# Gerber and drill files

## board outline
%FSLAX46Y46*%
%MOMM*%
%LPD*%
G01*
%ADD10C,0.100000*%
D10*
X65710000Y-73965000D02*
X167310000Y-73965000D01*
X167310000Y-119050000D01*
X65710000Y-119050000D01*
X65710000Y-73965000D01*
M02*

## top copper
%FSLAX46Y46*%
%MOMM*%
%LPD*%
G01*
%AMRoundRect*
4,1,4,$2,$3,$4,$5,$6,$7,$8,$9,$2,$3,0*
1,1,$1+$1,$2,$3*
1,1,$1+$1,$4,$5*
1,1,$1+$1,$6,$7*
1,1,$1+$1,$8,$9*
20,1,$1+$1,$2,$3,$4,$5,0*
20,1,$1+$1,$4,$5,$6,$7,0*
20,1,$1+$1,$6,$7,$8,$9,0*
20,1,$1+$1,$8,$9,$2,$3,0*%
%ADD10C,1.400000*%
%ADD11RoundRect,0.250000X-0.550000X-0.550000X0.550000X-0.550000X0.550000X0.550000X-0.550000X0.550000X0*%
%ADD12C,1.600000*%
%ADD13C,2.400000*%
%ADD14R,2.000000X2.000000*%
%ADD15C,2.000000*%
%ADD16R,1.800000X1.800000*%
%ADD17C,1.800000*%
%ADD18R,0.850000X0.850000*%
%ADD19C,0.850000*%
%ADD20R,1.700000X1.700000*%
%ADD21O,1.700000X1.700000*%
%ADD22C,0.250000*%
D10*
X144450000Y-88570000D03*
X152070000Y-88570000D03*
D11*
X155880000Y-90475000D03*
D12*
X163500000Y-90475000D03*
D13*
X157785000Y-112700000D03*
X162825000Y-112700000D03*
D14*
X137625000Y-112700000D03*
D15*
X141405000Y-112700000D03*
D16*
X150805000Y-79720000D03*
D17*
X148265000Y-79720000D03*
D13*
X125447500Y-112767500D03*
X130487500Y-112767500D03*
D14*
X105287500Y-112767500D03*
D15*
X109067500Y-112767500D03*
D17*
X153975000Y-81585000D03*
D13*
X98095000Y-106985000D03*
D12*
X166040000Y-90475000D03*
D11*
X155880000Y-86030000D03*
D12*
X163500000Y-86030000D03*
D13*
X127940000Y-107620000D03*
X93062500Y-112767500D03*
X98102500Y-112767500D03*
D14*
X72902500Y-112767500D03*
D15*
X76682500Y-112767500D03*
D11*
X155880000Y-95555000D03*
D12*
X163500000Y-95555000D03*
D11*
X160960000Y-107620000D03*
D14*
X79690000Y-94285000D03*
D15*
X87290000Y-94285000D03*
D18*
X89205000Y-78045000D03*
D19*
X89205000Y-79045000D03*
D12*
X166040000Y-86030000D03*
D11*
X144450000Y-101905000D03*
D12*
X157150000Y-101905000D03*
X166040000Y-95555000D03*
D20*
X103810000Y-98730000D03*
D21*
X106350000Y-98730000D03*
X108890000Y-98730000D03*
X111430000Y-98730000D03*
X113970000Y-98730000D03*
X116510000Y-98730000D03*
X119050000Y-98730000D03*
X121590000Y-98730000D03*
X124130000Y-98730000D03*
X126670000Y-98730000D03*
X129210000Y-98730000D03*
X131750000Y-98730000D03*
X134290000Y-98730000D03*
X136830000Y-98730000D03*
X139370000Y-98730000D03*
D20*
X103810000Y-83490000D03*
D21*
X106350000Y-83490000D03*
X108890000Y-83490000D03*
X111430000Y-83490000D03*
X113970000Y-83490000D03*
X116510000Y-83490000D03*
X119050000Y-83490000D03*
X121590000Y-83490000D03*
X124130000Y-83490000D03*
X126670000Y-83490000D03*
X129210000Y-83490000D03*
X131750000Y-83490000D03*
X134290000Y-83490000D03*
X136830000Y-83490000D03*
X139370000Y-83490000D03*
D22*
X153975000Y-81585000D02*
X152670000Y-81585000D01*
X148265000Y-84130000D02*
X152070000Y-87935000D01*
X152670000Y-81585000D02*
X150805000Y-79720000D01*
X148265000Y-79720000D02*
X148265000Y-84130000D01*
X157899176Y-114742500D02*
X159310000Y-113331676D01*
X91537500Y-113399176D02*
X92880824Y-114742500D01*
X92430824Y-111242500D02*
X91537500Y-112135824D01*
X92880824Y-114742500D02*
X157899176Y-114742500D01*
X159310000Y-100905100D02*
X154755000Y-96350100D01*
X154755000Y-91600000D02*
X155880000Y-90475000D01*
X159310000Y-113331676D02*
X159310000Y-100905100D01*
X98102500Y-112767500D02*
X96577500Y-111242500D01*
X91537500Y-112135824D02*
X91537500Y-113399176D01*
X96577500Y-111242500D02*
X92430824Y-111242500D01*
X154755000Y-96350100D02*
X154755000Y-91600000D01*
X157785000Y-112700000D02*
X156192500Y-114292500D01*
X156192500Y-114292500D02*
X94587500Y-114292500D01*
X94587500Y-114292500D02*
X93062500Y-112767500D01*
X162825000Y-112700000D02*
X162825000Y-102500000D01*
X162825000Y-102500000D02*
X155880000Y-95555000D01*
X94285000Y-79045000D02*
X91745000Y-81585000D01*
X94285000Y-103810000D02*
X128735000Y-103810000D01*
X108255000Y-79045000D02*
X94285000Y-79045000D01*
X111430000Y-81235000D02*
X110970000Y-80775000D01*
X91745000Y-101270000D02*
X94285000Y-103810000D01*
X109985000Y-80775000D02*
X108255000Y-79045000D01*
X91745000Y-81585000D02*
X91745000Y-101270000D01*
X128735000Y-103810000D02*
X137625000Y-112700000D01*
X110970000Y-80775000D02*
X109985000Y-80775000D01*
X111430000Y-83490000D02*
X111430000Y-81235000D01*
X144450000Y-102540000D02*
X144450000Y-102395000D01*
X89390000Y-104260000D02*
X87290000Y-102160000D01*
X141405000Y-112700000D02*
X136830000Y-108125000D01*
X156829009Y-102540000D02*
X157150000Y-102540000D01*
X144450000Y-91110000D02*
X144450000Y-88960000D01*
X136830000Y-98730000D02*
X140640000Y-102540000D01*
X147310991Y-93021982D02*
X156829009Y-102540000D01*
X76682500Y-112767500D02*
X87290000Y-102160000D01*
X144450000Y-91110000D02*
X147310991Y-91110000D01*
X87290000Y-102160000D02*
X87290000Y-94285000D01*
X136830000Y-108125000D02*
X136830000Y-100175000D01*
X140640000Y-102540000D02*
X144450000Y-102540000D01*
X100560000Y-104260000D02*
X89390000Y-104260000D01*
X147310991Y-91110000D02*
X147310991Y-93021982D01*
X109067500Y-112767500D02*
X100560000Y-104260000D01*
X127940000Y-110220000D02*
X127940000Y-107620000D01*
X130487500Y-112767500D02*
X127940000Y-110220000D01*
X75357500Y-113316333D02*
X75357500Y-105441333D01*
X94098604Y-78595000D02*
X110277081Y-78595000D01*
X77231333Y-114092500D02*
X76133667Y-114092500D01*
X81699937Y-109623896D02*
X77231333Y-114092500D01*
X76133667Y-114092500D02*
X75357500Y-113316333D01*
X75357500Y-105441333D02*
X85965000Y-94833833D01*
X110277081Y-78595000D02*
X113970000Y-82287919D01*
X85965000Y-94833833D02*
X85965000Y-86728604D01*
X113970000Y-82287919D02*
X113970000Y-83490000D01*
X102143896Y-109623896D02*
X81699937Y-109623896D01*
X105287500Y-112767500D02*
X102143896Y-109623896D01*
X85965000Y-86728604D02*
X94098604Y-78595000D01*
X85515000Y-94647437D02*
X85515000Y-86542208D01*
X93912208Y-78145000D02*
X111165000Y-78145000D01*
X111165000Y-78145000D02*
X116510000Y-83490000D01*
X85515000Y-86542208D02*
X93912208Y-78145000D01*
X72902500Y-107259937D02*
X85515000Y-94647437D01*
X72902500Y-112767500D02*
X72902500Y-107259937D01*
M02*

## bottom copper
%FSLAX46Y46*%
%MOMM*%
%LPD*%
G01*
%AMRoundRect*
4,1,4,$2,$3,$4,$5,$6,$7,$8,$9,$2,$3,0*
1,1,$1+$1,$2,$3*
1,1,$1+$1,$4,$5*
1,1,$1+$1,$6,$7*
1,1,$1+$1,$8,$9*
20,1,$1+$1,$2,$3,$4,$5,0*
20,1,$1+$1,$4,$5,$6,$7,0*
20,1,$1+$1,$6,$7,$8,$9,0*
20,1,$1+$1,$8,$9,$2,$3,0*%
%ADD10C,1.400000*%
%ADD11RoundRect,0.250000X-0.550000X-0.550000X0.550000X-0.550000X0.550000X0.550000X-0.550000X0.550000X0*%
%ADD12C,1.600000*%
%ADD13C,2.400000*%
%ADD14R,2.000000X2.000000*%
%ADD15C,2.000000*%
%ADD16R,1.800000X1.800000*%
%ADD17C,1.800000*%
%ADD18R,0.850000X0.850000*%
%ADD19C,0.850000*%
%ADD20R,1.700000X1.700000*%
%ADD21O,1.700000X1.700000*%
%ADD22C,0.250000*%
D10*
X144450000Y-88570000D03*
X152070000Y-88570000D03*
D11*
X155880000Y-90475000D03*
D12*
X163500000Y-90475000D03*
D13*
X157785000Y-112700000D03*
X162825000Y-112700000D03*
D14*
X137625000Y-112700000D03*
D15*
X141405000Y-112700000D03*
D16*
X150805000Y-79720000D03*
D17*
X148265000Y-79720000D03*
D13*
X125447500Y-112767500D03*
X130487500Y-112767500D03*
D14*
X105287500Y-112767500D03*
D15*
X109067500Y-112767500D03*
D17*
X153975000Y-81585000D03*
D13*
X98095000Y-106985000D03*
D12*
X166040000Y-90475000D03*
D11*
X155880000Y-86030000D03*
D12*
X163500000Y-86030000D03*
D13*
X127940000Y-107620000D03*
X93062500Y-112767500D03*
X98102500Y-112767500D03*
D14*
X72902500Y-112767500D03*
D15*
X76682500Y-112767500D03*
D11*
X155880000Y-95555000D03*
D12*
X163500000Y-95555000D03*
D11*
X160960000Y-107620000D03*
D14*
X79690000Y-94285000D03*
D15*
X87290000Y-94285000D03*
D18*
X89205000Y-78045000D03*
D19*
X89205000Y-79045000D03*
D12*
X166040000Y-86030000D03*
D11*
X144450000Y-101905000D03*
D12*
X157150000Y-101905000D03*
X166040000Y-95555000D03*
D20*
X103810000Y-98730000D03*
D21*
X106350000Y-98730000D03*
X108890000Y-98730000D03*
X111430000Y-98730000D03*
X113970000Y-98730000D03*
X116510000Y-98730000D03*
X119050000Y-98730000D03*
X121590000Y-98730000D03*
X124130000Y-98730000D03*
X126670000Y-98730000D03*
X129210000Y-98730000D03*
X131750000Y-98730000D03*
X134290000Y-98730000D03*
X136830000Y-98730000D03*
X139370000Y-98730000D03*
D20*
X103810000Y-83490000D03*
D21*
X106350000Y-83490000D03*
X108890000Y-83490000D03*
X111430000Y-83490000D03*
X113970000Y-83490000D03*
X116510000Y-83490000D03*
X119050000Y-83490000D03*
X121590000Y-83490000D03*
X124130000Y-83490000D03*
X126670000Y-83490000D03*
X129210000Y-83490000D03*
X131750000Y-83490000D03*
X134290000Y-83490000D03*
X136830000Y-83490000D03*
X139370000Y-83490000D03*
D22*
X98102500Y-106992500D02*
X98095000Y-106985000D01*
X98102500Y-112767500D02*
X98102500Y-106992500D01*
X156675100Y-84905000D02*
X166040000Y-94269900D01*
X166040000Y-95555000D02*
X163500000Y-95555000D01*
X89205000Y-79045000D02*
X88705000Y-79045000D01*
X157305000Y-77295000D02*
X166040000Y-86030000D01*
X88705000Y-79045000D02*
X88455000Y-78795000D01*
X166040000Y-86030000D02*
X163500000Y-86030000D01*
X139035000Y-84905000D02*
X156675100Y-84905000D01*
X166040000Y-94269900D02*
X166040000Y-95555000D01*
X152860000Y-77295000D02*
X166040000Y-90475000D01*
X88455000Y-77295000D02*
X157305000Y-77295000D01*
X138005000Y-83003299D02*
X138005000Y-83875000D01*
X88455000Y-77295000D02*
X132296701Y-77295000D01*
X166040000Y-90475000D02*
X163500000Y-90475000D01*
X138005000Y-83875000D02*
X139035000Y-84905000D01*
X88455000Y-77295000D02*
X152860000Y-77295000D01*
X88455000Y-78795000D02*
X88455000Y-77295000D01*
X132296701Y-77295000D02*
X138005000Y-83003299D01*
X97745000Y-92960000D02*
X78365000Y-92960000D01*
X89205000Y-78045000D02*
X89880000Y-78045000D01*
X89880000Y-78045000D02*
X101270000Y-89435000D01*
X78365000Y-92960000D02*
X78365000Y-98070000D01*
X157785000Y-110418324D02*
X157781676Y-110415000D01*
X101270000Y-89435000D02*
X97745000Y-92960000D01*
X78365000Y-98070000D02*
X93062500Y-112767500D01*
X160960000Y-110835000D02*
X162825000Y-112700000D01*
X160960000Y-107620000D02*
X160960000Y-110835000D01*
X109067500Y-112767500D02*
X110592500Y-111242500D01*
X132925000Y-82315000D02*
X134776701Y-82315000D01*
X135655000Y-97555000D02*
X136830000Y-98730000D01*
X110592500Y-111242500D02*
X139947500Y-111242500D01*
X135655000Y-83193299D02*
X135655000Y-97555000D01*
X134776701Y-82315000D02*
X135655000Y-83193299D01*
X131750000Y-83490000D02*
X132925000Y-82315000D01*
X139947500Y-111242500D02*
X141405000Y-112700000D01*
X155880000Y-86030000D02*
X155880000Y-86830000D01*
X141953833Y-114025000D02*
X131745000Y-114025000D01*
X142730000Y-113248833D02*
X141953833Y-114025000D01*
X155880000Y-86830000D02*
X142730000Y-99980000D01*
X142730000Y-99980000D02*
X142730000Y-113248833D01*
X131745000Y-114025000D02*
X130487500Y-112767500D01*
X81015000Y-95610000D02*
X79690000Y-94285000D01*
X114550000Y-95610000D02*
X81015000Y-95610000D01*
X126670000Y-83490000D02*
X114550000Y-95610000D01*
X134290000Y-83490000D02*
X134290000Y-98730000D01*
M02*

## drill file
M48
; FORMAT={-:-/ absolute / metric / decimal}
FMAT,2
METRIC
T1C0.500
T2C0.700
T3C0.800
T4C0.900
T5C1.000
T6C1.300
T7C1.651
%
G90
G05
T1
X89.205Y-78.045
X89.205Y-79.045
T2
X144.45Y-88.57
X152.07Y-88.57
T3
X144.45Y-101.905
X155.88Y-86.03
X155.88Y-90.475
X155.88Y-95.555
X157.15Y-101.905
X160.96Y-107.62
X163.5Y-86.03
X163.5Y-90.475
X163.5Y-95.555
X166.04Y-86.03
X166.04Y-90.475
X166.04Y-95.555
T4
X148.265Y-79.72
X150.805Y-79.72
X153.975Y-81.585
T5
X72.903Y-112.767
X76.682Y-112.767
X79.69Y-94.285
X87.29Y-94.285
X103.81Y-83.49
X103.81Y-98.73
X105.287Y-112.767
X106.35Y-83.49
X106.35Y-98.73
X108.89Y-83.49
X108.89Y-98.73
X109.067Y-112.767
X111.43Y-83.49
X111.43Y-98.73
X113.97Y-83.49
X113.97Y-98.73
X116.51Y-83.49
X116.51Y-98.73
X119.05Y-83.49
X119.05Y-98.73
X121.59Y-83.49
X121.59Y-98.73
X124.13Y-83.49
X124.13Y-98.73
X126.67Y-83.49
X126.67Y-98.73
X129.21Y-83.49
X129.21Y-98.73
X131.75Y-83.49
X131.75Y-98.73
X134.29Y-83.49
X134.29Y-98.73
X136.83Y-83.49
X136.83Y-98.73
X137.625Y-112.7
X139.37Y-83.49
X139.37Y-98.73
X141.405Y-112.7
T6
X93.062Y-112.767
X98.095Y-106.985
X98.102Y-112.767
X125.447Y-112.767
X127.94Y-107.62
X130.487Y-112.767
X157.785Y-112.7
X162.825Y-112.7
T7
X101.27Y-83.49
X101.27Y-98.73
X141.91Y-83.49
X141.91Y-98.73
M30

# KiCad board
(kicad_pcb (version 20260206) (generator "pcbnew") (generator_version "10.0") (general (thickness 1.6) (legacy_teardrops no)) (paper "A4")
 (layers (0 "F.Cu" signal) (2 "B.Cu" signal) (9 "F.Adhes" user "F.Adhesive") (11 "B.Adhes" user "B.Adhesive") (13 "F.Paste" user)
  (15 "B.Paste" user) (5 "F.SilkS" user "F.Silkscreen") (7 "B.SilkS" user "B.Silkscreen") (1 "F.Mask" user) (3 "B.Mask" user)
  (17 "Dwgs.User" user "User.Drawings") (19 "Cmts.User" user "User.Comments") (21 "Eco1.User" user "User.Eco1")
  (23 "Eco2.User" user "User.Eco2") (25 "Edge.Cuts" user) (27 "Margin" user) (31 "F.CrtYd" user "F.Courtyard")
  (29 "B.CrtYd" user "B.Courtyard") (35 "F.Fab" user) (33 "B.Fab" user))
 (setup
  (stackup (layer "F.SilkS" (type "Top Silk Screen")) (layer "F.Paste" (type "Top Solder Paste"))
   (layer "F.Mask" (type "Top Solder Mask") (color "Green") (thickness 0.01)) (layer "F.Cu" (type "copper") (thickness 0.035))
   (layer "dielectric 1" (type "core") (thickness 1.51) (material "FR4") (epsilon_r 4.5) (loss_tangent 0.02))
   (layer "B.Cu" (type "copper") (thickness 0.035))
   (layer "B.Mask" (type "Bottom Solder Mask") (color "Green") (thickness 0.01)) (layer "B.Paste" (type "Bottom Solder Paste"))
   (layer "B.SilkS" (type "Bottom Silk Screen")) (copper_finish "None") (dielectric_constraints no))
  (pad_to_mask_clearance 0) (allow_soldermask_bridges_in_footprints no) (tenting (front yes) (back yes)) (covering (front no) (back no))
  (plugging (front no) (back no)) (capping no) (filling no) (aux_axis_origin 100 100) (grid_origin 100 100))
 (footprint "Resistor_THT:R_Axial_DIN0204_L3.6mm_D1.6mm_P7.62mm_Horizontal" (layer "F.Cu") (at 144.45 88.57)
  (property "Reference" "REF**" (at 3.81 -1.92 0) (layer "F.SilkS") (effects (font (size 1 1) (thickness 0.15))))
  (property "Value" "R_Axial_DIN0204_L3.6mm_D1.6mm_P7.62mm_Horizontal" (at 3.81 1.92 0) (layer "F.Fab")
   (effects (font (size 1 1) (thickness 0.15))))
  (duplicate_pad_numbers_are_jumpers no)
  (pad "1" thru_hole circle (at 0 0) (size 1.4 1.4) (drill 0.7) (layers "*.Cu" "*.Mask") (remove_unused_layers no))
  (pad "2" thru_hole circle (at 7.62 0) (size 1.4 1.4) (drill 0.7) (layers "*.Cu" "*.Mask") (remove_unused_layers no)))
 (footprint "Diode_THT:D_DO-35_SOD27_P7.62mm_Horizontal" (layer "F.Cu") (at 155.88 90.475)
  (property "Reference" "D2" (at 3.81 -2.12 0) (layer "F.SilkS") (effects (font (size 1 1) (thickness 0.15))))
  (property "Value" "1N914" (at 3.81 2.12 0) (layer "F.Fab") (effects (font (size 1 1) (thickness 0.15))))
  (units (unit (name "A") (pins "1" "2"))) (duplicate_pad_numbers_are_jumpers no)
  (pad "1" thru_hole roundrect (at 0 0) (size 1.6 1.6) (drill 0.8) (layers "*.Cu" "*.Mask") (remove_unused_layers no)
   (roundrect_rratio 0.15625) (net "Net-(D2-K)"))
  (pad "2" thru_hole circle (at 7.62 0) (size 1.6 1.6) (drill 0.8) (layers "*.Cu" "*.Mask") (remove_unused_layers no) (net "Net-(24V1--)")))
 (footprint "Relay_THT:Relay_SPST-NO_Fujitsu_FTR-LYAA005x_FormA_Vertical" (layer "F.Cu") (at 137.625 112.7)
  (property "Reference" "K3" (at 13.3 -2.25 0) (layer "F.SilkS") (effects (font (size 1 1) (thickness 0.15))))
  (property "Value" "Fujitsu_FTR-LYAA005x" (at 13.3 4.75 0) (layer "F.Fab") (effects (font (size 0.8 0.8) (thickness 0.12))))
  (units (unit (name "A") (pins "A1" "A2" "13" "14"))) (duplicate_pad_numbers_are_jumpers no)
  (pad "13" thru_hole circle (at 20.16 0) (size 2.4 2.4) (drill 1.3) (layers "*.Cu" "*.Mask") (remove_unused_layers no) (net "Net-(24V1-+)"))
  (pad "14" thru_hole circle (at 25.2 0) (size 2.4 2.4) (drill 1.3) (layers "*.Cu" "*.Mask") (remove_unused_layers no) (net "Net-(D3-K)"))
  (pad "A1" thru_hole rect (at 0 0) (size 2 2) (drill 1) (layers "*.Cu" "*.Mask") (remove_unused_layers no) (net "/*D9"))
  (pad "A2" thru_hole circle (at 3.78 0) (size 2 2) (drill 1) (layers "*.Cu" "*.Mask") (remove_unused_layers no) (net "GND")))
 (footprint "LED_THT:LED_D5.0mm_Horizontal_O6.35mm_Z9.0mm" (layer "F.Cu") (at 150.805 79.72 180)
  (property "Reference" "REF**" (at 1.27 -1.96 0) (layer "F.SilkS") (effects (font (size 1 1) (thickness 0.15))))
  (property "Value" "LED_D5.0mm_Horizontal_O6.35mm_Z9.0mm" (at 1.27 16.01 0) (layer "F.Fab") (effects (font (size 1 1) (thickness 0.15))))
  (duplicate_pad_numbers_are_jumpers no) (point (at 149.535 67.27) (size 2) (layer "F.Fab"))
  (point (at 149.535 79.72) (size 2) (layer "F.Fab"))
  (pad "1" thru_hole rect (at 0 0 180) (size 1.8 1.8) (drill 0.9) (layers "*.Cu" "*.Mask") (remove_unused_layers no))
  (pad "2" thru_hole circle (at 2.54 0 180) (size 1.8 1.8) (drill 0.9) (layers "*.Cu" "*.Mask") (remove_unused_layers no)))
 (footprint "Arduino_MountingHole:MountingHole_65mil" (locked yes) (layer "F.Cu") (at 101.27 83.49)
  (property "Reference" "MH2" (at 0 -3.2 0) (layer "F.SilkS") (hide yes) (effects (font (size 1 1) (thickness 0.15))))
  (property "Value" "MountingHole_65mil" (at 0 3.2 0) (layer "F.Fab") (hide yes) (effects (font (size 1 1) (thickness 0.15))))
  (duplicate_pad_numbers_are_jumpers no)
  (pad "" np_thru_hole circle (at 0 0) (size 1.651 1.651) (drill 1.651) (layers "*.Cu" "*.Mask")))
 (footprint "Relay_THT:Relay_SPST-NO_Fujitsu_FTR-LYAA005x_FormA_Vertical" (layer "F.Cu") (at 105.2875 112.7675)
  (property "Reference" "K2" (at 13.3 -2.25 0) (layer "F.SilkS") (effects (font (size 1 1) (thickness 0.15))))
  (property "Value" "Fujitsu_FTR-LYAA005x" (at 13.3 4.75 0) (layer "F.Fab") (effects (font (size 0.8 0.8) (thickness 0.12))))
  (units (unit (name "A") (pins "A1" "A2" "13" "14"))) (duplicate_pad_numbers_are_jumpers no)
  (pad "13" thru_hole circle (at 20.16 0) (size 2.4 2.4) (drill 1.3) (layers "*.Cu" "*.Mask") (remove_unused_layers no)
   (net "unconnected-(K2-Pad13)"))
  (pad "14" thru_hole circle (at 25.2 0) (size 2.4 2.4) (drill 1.3) (layers "*.Cu" "*.Mask") (remove_unused_layers no) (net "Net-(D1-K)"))
  (pad "A1" thru_hole rect (at 0 0) (size 2 2) (drill 1) (layers "*.Cu" "*.Mask") (remove_unused_layers no) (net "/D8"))
  (pad "A2" thru_hole circle (at 3.78 0) (size 2 2) (drill 1) (layers "*.Cu" "*.Mask") (remove_unused_layers no) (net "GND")))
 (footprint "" (layer "F.Cu") (at 153.975 81.585)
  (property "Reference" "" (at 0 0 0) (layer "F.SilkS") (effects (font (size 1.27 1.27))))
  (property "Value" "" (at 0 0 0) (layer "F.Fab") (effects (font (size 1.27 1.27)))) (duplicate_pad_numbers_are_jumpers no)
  (pad "2" thru_hole circle (at 0 0 180) (size 1.8 1.8) (drill 0.9) (layers "*.Cu" "*.Mask") (remove_unused_layers no)))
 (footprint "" (layer "F.Cu") (at 98.095 106.985)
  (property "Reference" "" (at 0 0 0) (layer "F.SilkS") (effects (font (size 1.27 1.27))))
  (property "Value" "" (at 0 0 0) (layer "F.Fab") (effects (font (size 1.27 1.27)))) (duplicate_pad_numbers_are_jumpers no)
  (pad "14" thru_hole circle (at 0 0) (size 2.4 2.4) (drill 1.3) (layers "*.Cu" "*.Mask") (remove_unused_layers no) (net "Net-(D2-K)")))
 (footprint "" (layer "F.Cu") (at 166.04 90.475)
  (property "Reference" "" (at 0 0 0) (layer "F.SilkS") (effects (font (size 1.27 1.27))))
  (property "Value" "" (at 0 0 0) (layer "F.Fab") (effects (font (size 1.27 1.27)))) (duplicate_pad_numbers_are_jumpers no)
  (pad "2" thru_hole circle (at 0 0) (size 1.6 1.6) (drill 0.8) (layers "*.Cu" "*.Mask") (remove_unused_layers no) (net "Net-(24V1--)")))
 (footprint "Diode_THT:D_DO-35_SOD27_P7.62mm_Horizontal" (layer "F.Cu") (at 155.88 86.03)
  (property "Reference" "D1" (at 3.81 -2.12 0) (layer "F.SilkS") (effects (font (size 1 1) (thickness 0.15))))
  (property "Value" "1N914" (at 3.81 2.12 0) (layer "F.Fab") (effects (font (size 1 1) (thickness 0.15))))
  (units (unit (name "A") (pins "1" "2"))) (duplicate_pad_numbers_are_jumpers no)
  (pad "1" thru_hole roundrect (at 0 0) (size 1.6 1.6) (drill 0.8) (layers "*.Cu" "*.Mask") (remove_unused_layers no)
   (roundrect_rratio 0.15625) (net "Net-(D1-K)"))
  (pad "2" thru_hole circle (at 7.62 0) (size 1.6 1.6) (drill 0.8) (layers "*.Cu" "*.Mask") (remove_unused_layers no) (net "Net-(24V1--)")))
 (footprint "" (layer "F.Cu") (at 127.94 107.62)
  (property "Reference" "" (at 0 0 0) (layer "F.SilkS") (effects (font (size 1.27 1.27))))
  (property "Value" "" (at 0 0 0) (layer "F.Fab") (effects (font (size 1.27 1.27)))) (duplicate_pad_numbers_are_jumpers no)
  (pad "14" thru_hole circle (at 0 0) (size 2.4 2.4) (drill 1.3) (layers "*.Cu" "*.Mask") (remove_unused_layers no) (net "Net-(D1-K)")))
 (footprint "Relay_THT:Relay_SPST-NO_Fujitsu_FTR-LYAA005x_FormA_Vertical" (layer "F.Cu") (at 72.9025 112.7675)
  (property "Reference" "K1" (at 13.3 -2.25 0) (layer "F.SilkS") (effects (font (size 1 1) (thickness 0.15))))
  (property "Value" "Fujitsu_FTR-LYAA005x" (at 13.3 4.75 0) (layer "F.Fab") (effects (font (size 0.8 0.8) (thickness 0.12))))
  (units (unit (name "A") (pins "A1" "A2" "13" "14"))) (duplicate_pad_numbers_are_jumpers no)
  (pad "13" thru_hole circle (at 20.16 0) (size 2.4 2.4) (drill 1.3) (layers "*.Cu" "*.Mask") (remove_unused_layers no) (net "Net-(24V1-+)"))
  (pad "14" thru_hole circle (at 25.2 0) (size 2.4 2.4) (drill 1.3) (layers "*.Cu" "*.Mask") (remove_unused_layers no) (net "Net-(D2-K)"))
  (pad "A1" thru_hole rect (at 0 0) (size 2 2) (drill 1) (layers "*.Cu" "*.Mask") (remove_unused_layers no) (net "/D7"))
  (pad "A2" thru_hole circle (at 3.78 0) (size 2 2) (drill 1) (layers "*.Cu" "*.Mask") (remove_unused_layers no) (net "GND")))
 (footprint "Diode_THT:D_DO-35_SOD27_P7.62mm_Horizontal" (layer "F.Cu") (at 155.88 95.555)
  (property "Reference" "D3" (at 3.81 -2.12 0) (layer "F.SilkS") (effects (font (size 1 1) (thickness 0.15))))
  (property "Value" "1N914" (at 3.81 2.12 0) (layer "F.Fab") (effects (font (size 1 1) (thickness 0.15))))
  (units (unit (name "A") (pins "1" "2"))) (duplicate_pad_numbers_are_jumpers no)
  (pad "1" thru_hole roundrect (at 0 0) (size 1.6 1.6) (drill 0.8) (layers "*.Cu" "*.Mask") (remove_unused_layers no)
   (roundrect_rratio 0.15625) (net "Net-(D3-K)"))
  (pad "2" thru_hole circle (at 7.62 0) (size 1.6 1.6) (drill 0.8) (layers "*.Cu" "*.Mask") (remove_unused_layers no) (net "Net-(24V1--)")))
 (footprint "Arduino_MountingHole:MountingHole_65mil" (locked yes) (layer "F.Cu") (at 141.91 98.73)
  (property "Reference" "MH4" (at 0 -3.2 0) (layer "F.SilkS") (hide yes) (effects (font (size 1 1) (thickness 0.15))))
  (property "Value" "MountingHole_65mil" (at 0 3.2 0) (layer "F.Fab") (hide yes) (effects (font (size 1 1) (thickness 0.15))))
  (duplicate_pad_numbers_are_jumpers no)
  (pad "" np_thru_hole circle (at 0 0) (size 1.651 1.651) (drill 1.651) (layers "*.Cu" "*.Mask")))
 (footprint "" (layer "F.Cu") (at 160.96 107.62)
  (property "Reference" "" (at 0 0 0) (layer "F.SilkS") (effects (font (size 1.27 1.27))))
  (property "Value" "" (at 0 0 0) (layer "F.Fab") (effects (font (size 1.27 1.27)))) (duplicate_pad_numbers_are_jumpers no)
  (pad "1" thru_hole roundrect (at 0 0) (size 1.6 1.6) (drill 0.8) (layers "*.Cu" "*.Mask") (remove_unused_layers no)
   (roundrect_rratio 0.15625) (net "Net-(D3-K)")))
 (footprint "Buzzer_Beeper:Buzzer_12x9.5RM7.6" (layer "F.Cu") (at 79.69 94.285)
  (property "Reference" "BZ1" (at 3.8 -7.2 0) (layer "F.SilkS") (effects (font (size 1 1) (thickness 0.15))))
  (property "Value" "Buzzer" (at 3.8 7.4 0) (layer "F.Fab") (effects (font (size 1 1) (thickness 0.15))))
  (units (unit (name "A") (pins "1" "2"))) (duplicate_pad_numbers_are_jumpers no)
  (pad "1" thru_hole rect (at 0 0) (size 2 2) (drill 1) (layers "*.Cu" "*.Mask") (remove_unused_layers no) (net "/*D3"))
  (pad "2" thru_hole circle (at 7.6 0) (size 2 2) (drill 1) (layers "*.Cu" "*.Mask") (remove_unused_layers no) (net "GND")))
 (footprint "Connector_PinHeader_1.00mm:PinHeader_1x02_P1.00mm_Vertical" (layer "F.Cu") (at 89.205 78.045)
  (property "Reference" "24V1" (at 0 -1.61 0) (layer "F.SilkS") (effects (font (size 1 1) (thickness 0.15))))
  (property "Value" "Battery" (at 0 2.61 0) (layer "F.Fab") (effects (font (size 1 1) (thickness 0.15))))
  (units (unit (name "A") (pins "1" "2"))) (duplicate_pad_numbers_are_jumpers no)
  (pad "1" thru_hole rect (at 0 0) (size 0.85 0.85) (drill 0.5) (layers "*.Cu" "*.Mask") (remove_unused_layers no) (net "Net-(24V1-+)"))
  (pad "2" thru_hole circle (at 0 1) (size 0.85 0.85) (drill 0.5) (layers "*.Cu" "*.Mask") (remove_unused_layers no) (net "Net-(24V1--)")))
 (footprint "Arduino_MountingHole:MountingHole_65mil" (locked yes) (layer "F.Cu") (at 101.27 98.73)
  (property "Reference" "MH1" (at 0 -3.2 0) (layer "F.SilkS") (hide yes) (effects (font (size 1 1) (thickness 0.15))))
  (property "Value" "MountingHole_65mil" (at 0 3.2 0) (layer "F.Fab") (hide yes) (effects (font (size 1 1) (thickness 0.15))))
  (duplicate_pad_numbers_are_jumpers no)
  (pad "" np_thru_hole circle (at 0 0) (size 1.651 1.651) (drill 1.651) (layers "*.Cu" "*.Mask")))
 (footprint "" (layer "F.Cu") (at 166.04 86.03)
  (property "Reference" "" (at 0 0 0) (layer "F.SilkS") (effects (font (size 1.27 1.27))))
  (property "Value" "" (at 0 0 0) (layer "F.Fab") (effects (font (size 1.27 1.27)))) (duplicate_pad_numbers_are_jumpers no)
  (pad "2" thru_hole circle (at 0 0) (size 1.6 1.6) (drill 0.8) (layers "*.Cu" "*.Mask") (remove_unused_layers no) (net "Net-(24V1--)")))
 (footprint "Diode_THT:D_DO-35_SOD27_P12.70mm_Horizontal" (layer "F.Cu") (at 144.45 101.905)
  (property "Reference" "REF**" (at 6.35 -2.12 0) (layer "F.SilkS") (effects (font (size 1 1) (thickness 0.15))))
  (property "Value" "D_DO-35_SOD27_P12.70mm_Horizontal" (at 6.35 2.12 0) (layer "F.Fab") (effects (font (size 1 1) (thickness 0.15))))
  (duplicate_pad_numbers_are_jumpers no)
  (pad "1" thru_hole roundrect (at 0 0) (size 1.6 1.6) (drill 0.8) (layers "*.Cu" "*.Mask") (remove_unused_layers no)
   (roundrect_rratio 0.15625))
  (pad "2" thru_hole circle (at 12.7 0) (size 1.6 1.6) (drill 0.8) (layers "*.Cu" "*.Mask") (remove_unused_layers no)))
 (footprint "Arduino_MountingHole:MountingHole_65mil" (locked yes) (layer "F.Cu") (at 141.91 83.49)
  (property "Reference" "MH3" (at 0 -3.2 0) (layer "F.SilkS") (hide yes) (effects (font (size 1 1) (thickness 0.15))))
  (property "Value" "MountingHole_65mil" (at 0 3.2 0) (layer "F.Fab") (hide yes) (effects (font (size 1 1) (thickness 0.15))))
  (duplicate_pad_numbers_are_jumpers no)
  (pad "" np_thru_hole circle (at 0 0) (size 1.651 1.651) (drill 1.651) (layers "*.Cu" "*.Mask")))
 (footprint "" (layer "F.Cu") (at 166.04 95.555)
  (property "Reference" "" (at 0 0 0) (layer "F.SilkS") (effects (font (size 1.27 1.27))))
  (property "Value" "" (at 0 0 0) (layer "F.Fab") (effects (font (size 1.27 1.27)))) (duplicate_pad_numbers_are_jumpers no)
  (pad "2" thru_hole circle (at 0 0) (size 1.6 1.6) (drill 0.8) (layers "*.Cu" "*.Mask") (remove_unused_layers no) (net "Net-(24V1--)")))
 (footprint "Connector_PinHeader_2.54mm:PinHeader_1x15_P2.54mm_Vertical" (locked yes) (layer "B.Cu") (at 103.81 98.73 -90)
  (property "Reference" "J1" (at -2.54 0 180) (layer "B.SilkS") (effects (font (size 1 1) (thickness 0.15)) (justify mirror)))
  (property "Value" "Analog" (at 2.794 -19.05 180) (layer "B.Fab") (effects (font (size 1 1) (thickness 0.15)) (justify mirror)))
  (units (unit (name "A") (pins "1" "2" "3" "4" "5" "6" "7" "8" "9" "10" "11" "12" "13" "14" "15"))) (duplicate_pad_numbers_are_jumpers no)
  (pad "1" thru_hole rect (at 0 0 270) (size 1.7 1.7) (drill 1) (layers "*.Cu" "*.Mask") (remove_unused_layers no) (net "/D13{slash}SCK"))
  (pad "2" thru_hole oval (at 0 -2.54 270) (size 1.7 1.7) (drill 1) (layers "*.Cu" "*.Mask") (remove_unused_layers no) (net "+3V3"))
  (pad "3" thru_hole oval (at 0 -5.08 270) (size 1.7 1.7) (drill 1) (layers "*.Cu" "*.Mask") (remove_unused_layers no) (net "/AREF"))
  (pad "4" thru_hole oval (at 0 -7.62 270) (size 1.7 1.7) (drill 1) (layers "*.Cu" "*.Mask") (remove_unused_layers no) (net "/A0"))
  (pad "5" thru_hole oval (at 0 -10.16 270) (size 1.7 1.7) (drill 1) (layers "*.Cu" "*.Mask") (remove_unused_layers no) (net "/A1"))
  (pad "6" thru_hole oval (at 0 -12.7 270) (size 1.7 1.7) (drill 1) (layers "*.Cu" "*.Mask") (remove_unused_layers no) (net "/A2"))
  (pad "7" thru_hole oval (at 0 -15.24 270) (size 1.7 1.7) (drill 1) (layers "*.Cu" "*.Mask") (remove_unused_layers no) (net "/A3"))
  (pad "8" thru_hole oval (at 0 -17.78 270) (size 1.7 1.7) (drill 1) (layers "*.Cu" "*.Mask") (remove_unused_layers no)
   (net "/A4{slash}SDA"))
  (pad "9" thru_hole oval (at 0 -20.32 270) (size 1.7 1.7) (drill 1) (layers "*.Cu" "*.Mask") (remove_unused_layers no)
   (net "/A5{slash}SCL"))
  (pad "10" thru_hole oval (at 0 -22.86 270) (size 1.7 1.7) (drill 1) (layers "*.Cu" "*.Mask") (remove_unused_layers no) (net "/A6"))
  (pad "11" thru_hole oval (at 0 -25.4 270) (size 1.7 1.7) (drill 1) (layers "*.Cu" "*.Mask") (remove_unused_layers no) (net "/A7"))
  (pad "12" thru_hole oval (at 0 -27.94 270) (size 1.7 1.7) (drill 1) (layers "*.Cu" "*.Mask") (remove_unused_layers no) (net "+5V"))
  (pad "13" thru_hole oval (at 0 -30.48 270) (size 1.7 1.7) (drill 1) (layers "*.Cu" "*.Mask") (remove_unused_layers no) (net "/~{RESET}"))
  (pad "14" thru_hole oval (at 0 -33.02 270) (size 1.7 1.7) (drill 1) (layers "*.Cu" "*.Mask") (remove_unused_layers no) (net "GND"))
  (pad "15" thru_hole oval (at 0 -35.56 270) (size 1.7 1.7) (drill 1) (layers "*.Cu" "*.Mask") (remove_unused_layers no) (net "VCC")))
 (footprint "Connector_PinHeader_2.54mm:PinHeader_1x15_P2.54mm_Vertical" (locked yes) (layer "B.Cu") (at 103.81 83.49 -90)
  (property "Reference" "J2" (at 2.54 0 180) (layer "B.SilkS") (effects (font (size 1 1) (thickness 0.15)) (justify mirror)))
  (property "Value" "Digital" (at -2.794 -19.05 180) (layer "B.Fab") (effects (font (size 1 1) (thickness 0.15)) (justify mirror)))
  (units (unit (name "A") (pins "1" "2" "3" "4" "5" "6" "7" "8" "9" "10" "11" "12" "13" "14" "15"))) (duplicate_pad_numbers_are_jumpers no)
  (pad "1" thru_hole rect (at 0 0 270) (size 1.7 1.7) (drill 1) (layers "*.Cu" "*.Mask") (remove_unused_layers no) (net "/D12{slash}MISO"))
  (pad "2" thru_hole oval (at 0 -2.54 270) (size 1.7 1.7) (drill 1) (layers "*.Cu" "*.Mask") (remove_unused_layers no)
   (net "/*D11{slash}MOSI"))
  (pad "3" thru_hole oval (at 0 -5.08 270) (size 1.7 1.7) (drill 1) (layers "*.Cu" "*.Mask") (remove_unused_layers no)
   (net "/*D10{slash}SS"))
  (pad "4" thru_hole oval (at 0 -7.62 270) (size 1.7 1.7) (drill 1) (layers "*.Cu" "*.Mask") (remove_unused_layers no) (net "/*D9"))
  (pad "5" thru_hole oval (at 0 -10.16 270) (size 1.7 1.7) (drill 1) (layers "*.Cu" "*.Mask") (remove_unused_layers no) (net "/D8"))
  (pad "6" thru_hole oval (at 0 -12.7 270) (size 1.7 1.7) (drill 1) (layers "*.Cu" "*.Mask") (remove_unused_layers no) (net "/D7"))
  (pad "7" thru_hole oval (at 0 -15.24 270) (size 1.7 1.7) (drill 1) (layers "*.Cu" "*.Mask") (remove_unused_layers no) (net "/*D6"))
  (pad "8" thru_hole oval (at 0 -17.78 270) (size 1.7 1.7) (drill 1) (layers "*.Cu" "*.Mask") (remove_unused_layers no) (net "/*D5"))
  (pad "9" thru_hole oval (at 0 -20.32 270) (size 1.7 1.7) (drill 1) (layers "*.Cu" "*.Mask") (remove_unused_layers no) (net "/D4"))
  (pad "10" thru_hole oval (at 0 -22.86 270) (size 1.7 1.7) (drill 1) (layers "*.Cu" "*.Mask") (remove_unused_layers no) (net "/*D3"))
  (pad "11" thru_hole oval (at 0 -25.4 270) (size 1.7 1.7) (drill 1) (layers "*.Cu" "*.Mask") (remove_unused_layers no) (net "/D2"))
  (pad "12" thru_hole oval (at 0 -27.94 270) (size 1.7 1.7) (drill 1) (layers "*.Cu" "*.Mask") (remove_unused_layers no) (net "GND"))
  (pad "13" thru_hole oval (at 0 -30.48 270) (size 1.7 1.7) (drill 1) (layers "*.Cu" "*.Mask") (remove_unused_layers no) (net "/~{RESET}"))
  (pad "14" thru_hole oval (at 0 -33.02 270) (size 1.7 1.7) (drill 1) (layers "*.Cu" "*.Mask") (remove_unused_layers no)
   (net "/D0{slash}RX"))
  (pad "15" thru_hole oval (at 0 -35.56 270) (size 1.7 1.7) (drill 1) (layers "*.Cu" "*.Mask") (remove_unused_layers no)
   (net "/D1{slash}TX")))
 (gr_rect (start 65.71 73.965) (end 167.31 119.05) (stroke (width 0.1) (type default)) (fill no) (layer "Edge.Cuts"))
 (segment (start 153.975 81.585) (end 152.67 81.585) (width 0.25) (layer "F.Cu") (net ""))
 (segment (start 148.265 84.13) (end 152.07 87.935) (width 0.25) (layer "F.Cu") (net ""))
 (segment (start 152.67 81.585) (end 150.805 79.72) (width 0.25) (layer "F.Cu") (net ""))
 (segment (start 148.265 79.72) (end 148.265 84.13) (width 0.25) (layer "F.Cu") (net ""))
 (segment (start 157.899176 114.7425) (end 159.31 113.331676) (width 0.25) (layer "F.Cu") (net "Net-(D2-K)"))
 (segment (start 91.5375 113.399176) (end 92.880824 114.7425) (width 0.25) (layer "F.Cu") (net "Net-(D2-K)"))
 (segment (start 92.430824 111.2425) (end 91.5375 112.135824) (width 0.25) (layer "F.Cu") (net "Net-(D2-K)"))
 (segment (start 92.880824 114.7425) (end 157.899176 114.7425) (width 0.25) (layer "F.Cu") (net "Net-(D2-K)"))
 (segment (start 159.31 100.9051) (end 154.755 96.3501) (width 0.25) (layer "F.Cu") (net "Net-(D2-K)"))
 (segment (start 154.755 91.6) (end 155.88 90.475) (width 0.25) (layer "F.Cu") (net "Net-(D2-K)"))
 (segment (start 159.31 113.331676) (end 159.31 100.9051) (width 0.25) (layer "F.Cu") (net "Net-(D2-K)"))
 (segment (start 98.1025 112.7675) (end 96.5775 111.2425) (width 0.25) (layer "F.Cu") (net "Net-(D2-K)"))
 (segment (start 91.5375 112.135824) (end 91.5375 113.399176) (width 0.25) (layer "F.Cu") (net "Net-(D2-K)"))
 (segment (start 96.5775 111.2425) (end 92.430824 111.2425) (width 0.25) (layer "F.Cu") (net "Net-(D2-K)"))
 (segment (start 154.755 96.3501) (end 154.755 91.6) (width 0.25) (layer "F.Cu") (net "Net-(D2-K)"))
 (segment (start 98.1025 106.9925) (end 98.095 106.985) (width 0.25) (layer "B.Cu") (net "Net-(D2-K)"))
 (segment (start 98.1025 112.7675) (end 98.1025 106.9925) (width 0.25) (layer "B.Cu") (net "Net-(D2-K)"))
 (segment (start 156.6751 84.905) (end 166.04 94.2699) (width 0.25) (layer "B.Cu") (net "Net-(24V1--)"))
 (segment (start 166.04 95.555) (end 163.5 95.555) (width 0.25) (layer "B.Cu") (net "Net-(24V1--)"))
 (segment (start 89.205 79.045) (end 88.705 79.045) (width 0.25) (layer "B.Cu") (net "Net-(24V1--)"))
 (segment (start 157.305 77.295) (end 166.04 86.03) (width 0.25) (layer "B.Cu") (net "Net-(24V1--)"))
 (segment (start 88.705 79.045) (end 88.455 78.795) (width 0.25) (layer "B.Cu") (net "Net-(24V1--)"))
 (segment (start 166.04 86.03) (end 163.5 86.03) (width 0.25) (layer "B.Cu") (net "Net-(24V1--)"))
 (segment (start 139.035 84.905) (end 156.6751 84.905) (width 0.25) (layer "B.Cu") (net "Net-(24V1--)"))
 (segment (start 166.04 94.2699) (end 166.04 95.555) (width 0.25) (layer "B.Cu") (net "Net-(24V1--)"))
 (segment (start 152.86 77.295) (end 166.04 90.475) (width 0.25) (layer "B.Cu") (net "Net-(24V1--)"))
 (segment (start 88.455 77.295) (end 157.305 77.295) (width 0.25) (layer "B.Cu") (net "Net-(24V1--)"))
 (segment (start 138.005 83.003299) (end 138.005 83.875) (width 0.25) (layer "B.Cu") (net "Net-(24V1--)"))
 (segment (start 88.455 77.295) (end 132.296701 77.295) (width 0.25) (layer "B.Cu") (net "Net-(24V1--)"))
 (segment (start 166.04 90.475) (end 163.5 90.475) (width 0.25) (layer "B.Cu") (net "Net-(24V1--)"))
 (segment (start 138.005 83.875) (end 139.035 84.905) (width 0.25) (layer "B.Cu") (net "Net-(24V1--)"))
 (segment (start 88.455 77.295) (end 152.86 77.295) (width 0.25) (layer "B.Cu") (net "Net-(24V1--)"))
 (segment (start 88.455 78.795) (end 88.455 77.295) (width 0.25) (layer "B.Cu") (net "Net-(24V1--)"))
 (segment (start 132.296701 77.295) (end 138.005 83.003299) (width 0.25) (layer "B.Cu") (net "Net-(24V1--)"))
 (segment (start 157.785 112.7) (end 156.1925 114.2925) (width 0.25) (layer "F.Cu") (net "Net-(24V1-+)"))
 (segment (start 156.1925 114.2925) (end 94.5875 114.2925) (width 0.25) (layer "F.Cu") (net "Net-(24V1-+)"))
 (segment (start 94.5875 114.2925) (end 93.0625 112.7675) (width 0.25) (layer "F.Cu") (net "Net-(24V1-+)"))
 (segment (start 97.745 92.96) (end 78.365 92.96) (width 0.25) (layer "B.Cu") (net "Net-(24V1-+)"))
 (segment (start 89.205 78.045) (end 89.88 78.045) (width 0.25) (layer "B.Cu") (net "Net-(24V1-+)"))
 (segment (start 89.88 78.045) (end 101.27 89.435) (width 0.25) (layer "B.Cu") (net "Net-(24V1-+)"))
 (segment (start 78.365 92.96) (end 78.365 98.07) (width 0.25) (layer "B.Cu") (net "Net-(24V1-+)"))
 (segment (start 157.785 110.418324) (end 157.781676 110.415) (width 0.25) (layer "B.Cu") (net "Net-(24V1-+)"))
 (segment (start 101.27 89.435) (end 97.745 92.96) (width 0.25) (layer "B.Cu") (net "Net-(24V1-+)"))
 (segment (start 78.365 98.07) (end 93.0625 112.7675) (width 0.25) (layer "B.Cu") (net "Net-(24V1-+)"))
 (segment (start 162.825 112.7) (end 162.825 102.5) (width 0.25) (layer "F.Cu") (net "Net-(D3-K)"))
 (segment (start 162.825 102.5) (end 155.88 95.555) (width 0.25) (layer "F.Cu") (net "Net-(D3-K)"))
 (segment (start 160.96 110.835) (end 162.825 112.7) (width 0.25) (layer "B.Cu") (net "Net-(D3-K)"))
 (segment (start 160.96 107.62) (end 160.96 110.835) (width 0.25) (layer "B.Cu") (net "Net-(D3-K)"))
 (segment (start 94.285 79.045) (end 91.745 81.585) (width 0.25) (layer "F.Cu") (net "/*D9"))
 (segment (start 94.285 103.81) (end 128.735 103.81) (width 0.25) (layer "F.Cu") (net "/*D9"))
 (segment (start 108.255 79.045) (end 94.285 79.045) (width 0.25) (layer "F.Cu") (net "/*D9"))
 (segment (start 111.43 81.235) (end 110.97 80.775) (width 0.25) (layer "F.Cu") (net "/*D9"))
 (segment (start 91.745 101.27) (end 94.285 103.81) (width 0.25) (layer "F.Cu") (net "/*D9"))
 (segment (start 109.985 80.775) (end 108.255 79.045) (width 0.25) (layer "F.Cu") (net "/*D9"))
 (segment (start 91.745 81.585) (end 91.745 101.27) (width 0.25) (layer "F.Cu") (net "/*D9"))
 (segment (start 128.735 103.81) (end 137.625 112.7) (width 0.25) (layer "F.Cu") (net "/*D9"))
 (segment (start 110.97 80.775) (end 109.985 80.775) (width 0.25) (layer "F.Cu") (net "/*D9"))
 (segment (start 111.43 83.49) (end 111.43 81.235) (width 0.25) (layer "F.Cu") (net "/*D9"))
 (segment (start 144.45 102.54) (end 144.45 102.395) (width 0.25) (layer "F.Cu") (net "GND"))
 (segment (start 89.39 104.26) (end 87.29 102.16) (width 0.25) (layer "F.Cu") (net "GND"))
 (segment (start 141.405 112.7) (end 136.83 108.125) (width 0.25) (layer "F.Cu") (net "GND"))
 (segment (start 156.829009 102.54) (end 157.15 102.54) (width 0.25) (layer "F.Cu") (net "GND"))
 (segment (start 144.45 91.11) (end 144.45 88.96) (width 0.25) (layer "F.Cu") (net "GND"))
 (segment (start 136.83 98.73) (end 140.64 102.54) (width 0.25) (layer "F.Cu") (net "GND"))
 (segment (start 147.310991 93.021982) (end 156.829009 102.54) (width 0.25) (layer "F.Cu") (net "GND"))
 (segment (start 76.6825 112.7675) (end 87.29 102.16) (width 0.25) (layer "F.Cu") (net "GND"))
 (segment (start 144.45 91.11) (end 147.310991 91.11) (width 0.25) (layer "F.Cu") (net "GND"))
 (segment (start 87.29 102.16) (end 87.29 94.285) (width 0.25) (layer "F.Cu") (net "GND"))
 (segment (start 136.83 108.125) (end 136.83 100.175) (width 0.25) (layer "F.Cu") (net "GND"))
 (segment (start 140.64 102.54) (end 144.45 102.54) (width 0.25) (layer "F.Cu") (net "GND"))
 (segment (start 100.56 104.26) (end 89.39 104.26) (width 0.25) (layer "F.Cu") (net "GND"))
 (segment (start 147.310991 91.11) (end 147.310991 93.021982) (width 0.25) (layer "F.Cu") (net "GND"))
 (segment (start 109.0675 112.7675) (end 100.56 104.26) (width 0.25) (layer "F.Cu") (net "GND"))
 (segment (start 109.0675 112.7675) (end 110.5925 111.2425) (width 0.25) (layer "B.Cu") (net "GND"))
 (segment (start 132.925 82.315) (end 134.776701 82.315) (width 0.25) (layer "B.Cu") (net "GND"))
 (segment (start 135.655 97.555) (end 136.83 98.73) (width 0.25) (layer "B.Cu") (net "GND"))
 (segment (start 110.5925 111.2425) (end 139.9475 111.2425) (width 0.25) (layer "B.Cu") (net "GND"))
 (segment (start 135.655 83.193299) (end 135.655 97.555) (width 0.25) (layer "B.Cu") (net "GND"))
 (segment (start 134.776701 82.315) (end 135.655 83.193299) (width 0.25) (layer "B.Cu") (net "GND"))
 (segment (start 131.75 83.49) (end 132.925 82.315) (width 0.25) (layer "B.Cu") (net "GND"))
 (segment (start 139.9475 111.2425) (end 141.405 112.7) (width 0.25) (layer "B.Cu") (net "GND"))
 (segment (start 127.94 110.22) (end 127.94 107.62) (width 0.25) (layer "F.Cu") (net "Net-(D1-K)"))
 (segment (start 130.4875 112.7675) (end 127.94 110.22) (width 0.25) (layer "F.Cu") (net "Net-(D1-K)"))
 (segment (start 155.88 86.03) (end 155.88 86.83) (width 0.25) (layer "B.Cu") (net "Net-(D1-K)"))
 (segment (start 141.953833 114.025) (end 131.745 114.025) (width 0.25) (layer "B.Cu") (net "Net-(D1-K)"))
 (segment (start 142.73 113.248833) (end 141.953833 114.025) (width 0.25) (layer "B.Cu") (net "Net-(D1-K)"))
 (segment (start 155.88 86.83) (end 142.73 99.98) (width 0.25) (layer "B.Cu") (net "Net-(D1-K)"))
 (segment (start 142.73 99.98) (end 142.73 113.248833) (width 0.25) (layer "B.Cu") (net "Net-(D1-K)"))
 (segment (start 131.745 114.025) (end 130.4875 112.7675) (width 0.25) (layer "B.Cu") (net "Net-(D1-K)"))
 (segment (start 75.3575 113.316333) (end 75.3575 105.441333) (width 0.25) (layer "F.Cu") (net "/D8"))
 (segment (start 94.098604 78.595) (end 110.277081 78.595) (width 0.25) (layer "F.Cu") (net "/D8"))
 (segment (start 77.231333 114.0925) (end 76.133667 114.0925) (width 0.25) (layer "F.Cu") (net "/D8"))
 (segment (start 81.699937 109.623896) (end 77.231333 114.0925) (width 0.25) (layer "F.Cu") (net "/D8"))
 (segment (start 76.133667 114.0925) (end 75.3575 113.316333) (width 0.25) (layer "F.Cu") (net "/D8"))
 (segment (start 75.3575 105.441333) (end 85.965 94.833833) (width 0.25) (layer "F.Cu") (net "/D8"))
 (segment (start 110.277081 78.595) (end 113.97 82.287919) (width 0.25) (layer "F.Cu") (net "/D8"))
 (segment (start 85.965 94.833833) (end 85.965 86.728604) (width 0.25) (layer "F.Cu") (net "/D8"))
 (segment (start 113.97 82.287919) (end 113.97 83.49) (width 0.25) (layer "F.Cu") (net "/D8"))
 (segment (start 102.143896 109.623896) (end 81.699937 109.623896) (width 0.25) (layer "F.Cu") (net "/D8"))
 (segment (start 105.2875 112.7675) (end 102.143896 109.623896) (width 0.25) (layer "F.Cu") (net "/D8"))
 (segment (start 85.965 86.728604) (end 94.098604 78.595) (width 0.25) (layer "F.Cu") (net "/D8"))
 (segment (start 85.515 94.647437) (end 85.515 86.542208) (width 0.25) (layer "F.Cu") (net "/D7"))
 (segment (start 93.912208 78.145) (end 111.165 78.145) (width 0.25) (layer "F.Cu") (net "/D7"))
 (segment (start 111.165 78.145) (end 116.51 83.49) (width 0.25) (layer "F.Cu") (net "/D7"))
 (segment (start 85.515 86.542208) (end 93.912208 78.145) (width 0.25) (layer "F.Cu") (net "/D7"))
 (segment (start 72.9025 107.259937) (end 85.515 94.647437) (width 0.25) (layer "F.Cu") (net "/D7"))
 (segment (start 72.9025 112.7675) (end 72.9025 107.259937) (width 0.25) (layer "F.Cu") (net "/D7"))
 (segment (start 81.015 95.61) (end 79.69 94.285) (width 0.25) (layer "B.Cu") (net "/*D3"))
 (segment (start 114.55 95.61) (end 81.015 95.61) (width 0.25) (layer "B.Cu") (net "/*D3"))
 (segment (start 126.67 83.49) (end 114.55 95.61) (width 0.25) (layer "B.Cu") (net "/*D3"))
 (segment (start 134.29 83.49) (end 134.29 98.73) (width 0.25) (layer "B.Cu") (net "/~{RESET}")))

